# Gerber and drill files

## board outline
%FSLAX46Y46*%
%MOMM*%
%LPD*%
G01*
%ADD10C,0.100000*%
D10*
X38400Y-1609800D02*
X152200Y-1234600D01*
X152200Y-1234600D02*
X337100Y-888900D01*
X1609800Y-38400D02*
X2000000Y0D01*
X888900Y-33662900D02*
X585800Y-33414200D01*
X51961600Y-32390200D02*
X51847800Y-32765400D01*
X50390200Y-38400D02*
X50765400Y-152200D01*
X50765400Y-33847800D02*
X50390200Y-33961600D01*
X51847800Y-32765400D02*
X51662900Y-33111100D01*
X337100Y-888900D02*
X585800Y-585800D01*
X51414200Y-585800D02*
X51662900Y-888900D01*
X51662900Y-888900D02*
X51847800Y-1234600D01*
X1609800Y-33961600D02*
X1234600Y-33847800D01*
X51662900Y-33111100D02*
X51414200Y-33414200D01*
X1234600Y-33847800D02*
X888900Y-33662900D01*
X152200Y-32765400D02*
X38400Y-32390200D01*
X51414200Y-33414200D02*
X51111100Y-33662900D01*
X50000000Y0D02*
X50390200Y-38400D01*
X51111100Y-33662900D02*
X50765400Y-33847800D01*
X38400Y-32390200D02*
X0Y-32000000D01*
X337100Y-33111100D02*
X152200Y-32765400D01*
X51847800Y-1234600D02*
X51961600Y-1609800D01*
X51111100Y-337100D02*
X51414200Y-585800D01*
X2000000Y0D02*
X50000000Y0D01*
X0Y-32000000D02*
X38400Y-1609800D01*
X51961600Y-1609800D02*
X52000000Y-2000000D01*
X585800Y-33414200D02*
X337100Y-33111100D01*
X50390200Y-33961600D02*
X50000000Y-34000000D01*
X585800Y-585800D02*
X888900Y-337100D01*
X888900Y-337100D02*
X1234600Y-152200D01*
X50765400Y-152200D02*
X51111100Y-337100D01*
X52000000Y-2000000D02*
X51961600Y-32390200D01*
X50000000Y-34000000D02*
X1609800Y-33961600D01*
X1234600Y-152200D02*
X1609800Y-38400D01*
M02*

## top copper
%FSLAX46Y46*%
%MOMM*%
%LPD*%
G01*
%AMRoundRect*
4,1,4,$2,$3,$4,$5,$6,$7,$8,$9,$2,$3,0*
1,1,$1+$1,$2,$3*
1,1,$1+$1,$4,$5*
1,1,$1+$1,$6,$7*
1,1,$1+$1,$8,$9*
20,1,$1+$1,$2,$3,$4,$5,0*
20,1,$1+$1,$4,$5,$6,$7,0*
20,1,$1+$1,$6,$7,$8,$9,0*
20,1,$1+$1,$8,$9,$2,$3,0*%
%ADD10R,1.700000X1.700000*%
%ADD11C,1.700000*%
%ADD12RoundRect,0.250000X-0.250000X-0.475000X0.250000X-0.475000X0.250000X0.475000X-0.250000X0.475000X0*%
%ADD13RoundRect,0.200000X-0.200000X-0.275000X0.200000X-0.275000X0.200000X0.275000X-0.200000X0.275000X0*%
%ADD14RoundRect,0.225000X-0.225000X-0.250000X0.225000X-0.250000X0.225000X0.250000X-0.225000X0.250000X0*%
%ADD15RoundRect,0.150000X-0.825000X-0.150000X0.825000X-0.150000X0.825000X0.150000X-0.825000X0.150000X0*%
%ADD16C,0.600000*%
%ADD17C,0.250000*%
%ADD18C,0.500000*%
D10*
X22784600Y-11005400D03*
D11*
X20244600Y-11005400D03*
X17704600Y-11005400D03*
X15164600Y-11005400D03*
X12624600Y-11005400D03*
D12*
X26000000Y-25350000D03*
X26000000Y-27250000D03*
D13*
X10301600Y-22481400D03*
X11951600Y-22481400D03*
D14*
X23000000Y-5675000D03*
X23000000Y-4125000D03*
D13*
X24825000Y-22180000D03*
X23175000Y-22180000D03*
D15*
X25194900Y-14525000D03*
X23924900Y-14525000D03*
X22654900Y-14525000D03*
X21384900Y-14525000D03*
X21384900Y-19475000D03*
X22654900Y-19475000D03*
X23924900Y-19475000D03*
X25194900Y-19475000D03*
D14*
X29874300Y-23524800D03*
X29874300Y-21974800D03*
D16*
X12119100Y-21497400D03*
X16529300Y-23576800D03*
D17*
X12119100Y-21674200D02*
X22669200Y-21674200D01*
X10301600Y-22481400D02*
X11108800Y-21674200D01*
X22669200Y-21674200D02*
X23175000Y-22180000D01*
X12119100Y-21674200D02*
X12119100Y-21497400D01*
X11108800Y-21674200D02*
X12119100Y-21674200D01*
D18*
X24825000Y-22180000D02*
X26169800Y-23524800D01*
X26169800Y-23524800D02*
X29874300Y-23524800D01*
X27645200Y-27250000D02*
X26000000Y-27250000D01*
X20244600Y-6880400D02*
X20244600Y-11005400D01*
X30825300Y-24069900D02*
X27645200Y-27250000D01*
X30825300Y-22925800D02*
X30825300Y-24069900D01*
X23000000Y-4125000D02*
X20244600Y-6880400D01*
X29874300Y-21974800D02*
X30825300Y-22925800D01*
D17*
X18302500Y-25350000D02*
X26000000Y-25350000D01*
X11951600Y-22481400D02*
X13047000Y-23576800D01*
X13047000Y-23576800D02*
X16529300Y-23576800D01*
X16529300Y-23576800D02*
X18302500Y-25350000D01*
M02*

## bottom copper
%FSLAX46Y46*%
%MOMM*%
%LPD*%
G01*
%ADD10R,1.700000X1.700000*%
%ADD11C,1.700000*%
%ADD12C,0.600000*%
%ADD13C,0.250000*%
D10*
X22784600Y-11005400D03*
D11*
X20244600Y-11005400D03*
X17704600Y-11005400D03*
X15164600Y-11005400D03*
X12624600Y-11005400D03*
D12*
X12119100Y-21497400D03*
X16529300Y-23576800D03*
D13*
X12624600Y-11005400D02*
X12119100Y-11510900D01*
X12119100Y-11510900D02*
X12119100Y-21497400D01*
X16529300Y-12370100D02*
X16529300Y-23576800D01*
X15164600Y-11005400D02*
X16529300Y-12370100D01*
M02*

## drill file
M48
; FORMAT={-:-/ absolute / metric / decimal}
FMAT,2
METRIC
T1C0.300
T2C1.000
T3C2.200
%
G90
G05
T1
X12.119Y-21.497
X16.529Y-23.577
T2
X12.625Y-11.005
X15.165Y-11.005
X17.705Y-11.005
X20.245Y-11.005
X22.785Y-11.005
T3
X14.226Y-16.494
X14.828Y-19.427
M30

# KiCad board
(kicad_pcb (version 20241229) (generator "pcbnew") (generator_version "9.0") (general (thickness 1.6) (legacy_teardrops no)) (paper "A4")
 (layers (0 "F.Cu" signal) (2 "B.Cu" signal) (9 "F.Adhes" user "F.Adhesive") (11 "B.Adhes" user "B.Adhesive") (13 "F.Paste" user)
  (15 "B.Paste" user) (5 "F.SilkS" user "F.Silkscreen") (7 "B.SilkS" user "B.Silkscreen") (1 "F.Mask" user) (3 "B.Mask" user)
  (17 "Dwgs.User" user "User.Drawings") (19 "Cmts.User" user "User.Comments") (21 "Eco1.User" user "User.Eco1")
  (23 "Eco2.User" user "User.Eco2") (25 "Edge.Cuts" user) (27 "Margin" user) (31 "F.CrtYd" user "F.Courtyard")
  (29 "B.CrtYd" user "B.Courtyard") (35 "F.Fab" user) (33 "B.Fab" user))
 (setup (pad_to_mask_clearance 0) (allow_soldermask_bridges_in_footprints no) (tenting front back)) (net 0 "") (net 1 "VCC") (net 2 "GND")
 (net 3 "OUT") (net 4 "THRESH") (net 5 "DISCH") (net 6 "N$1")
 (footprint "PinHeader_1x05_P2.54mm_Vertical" (layer "F.Cu") (at 22.7846 11.0054 -90)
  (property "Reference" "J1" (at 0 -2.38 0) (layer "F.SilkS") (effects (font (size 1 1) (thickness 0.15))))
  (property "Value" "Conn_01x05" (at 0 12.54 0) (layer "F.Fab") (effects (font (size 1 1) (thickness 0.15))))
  (pad "1" thru_hole rect (at 0 0) (size 1.7 1.7) (drill 1) (layers "*.Cu" "*.Mask") (remove_unused_layers no) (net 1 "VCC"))
  (pad "2" thru_hole circle (at 0 2.54) (size 1.7 1.7) (drill 1) (layers "*.Cu" "*.Mask") (remove_unused_layers no) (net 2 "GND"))
  (pad "3" thru_hole circle (at 0 5.08) (size 1.7 1.7) (drill 1) (layers "*.Cu" "*.Mask") (remove_unused_layers no) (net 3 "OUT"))
  (pad "4" thru_hole circle (at 0 7.62) (size 1.7 1.7) (drill 1) (layers "*.Cu" "*.Mask") (remove_unused_layers no) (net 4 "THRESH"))
  (pad "5" thru_hole circle (at 0 10.16) (size 1.7 1.7) (drill 1) (layers "*.Cu" "*.Mask") (remove_unused_layers no) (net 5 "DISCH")))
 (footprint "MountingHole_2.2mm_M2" (layer "F.Cu") (at 14.8283 19.4265)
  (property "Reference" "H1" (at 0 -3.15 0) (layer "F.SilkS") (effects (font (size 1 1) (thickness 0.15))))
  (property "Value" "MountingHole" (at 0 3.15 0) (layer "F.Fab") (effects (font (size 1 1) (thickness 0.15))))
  (pad "" np_thru_hole circle (at 0 0) (size 2.2 2.2) (drill 2.2) (layers "*.Cu" "*.Mask")))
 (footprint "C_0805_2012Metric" (layer "F.Cu") (at 26 26.3 -90)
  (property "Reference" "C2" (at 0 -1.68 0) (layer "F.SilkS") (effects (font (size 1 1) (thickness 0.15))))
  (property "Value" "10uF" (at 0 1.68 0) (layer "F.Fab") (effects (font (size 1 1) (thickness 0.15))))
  (pad "1" smd roundrect (at -0.95 0) (size 1 1.45) (layers "F.Cu" "F.Mask" "F.Paste") (roundrect_rratio 0.25) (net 4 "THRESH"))
  (pad "2" smd roundrect (at 0.95 0) (size 1 1.45) (layers "F.Cu" "F.Mask" "F.Paste") (roundrect_rratio 0.25) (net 2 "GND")))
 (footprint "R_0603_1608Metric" (layer "F.Cu") (at 11.1266 22.4814)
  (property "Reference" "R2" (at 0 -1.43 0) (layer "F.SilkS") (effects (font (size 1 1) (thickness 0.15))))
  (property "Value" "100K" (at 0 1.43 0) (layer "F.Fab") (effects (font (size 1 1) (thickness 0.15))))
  (pad "1" smd roundrect (at -0.825 0) (size 0.8 0.95) (layers "F.Cu" "F.Mask" "F.Paste") (roundrect_rratio 0.25) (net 5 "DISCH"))
  (pad "2" smd roundrect (at 0.825 0) (size 0.8 0.95) (layers "F.Cu" "F.Mask" "F.Paste") (roundrect_rratio 0.25) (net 4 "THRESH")))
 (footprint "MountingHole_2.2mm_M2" (layer "F.Cu") (at 14.2257 16.4942)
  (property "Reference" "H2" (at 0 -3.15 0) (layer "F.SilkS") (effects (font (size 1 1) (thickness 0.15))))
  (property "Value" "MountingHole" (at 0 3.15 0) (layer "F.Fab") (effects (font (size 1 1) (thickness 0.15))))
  (pad "" np_thru_hole circle (at 0 0) (size 2.2 2.2) (drill 2.2) (layers "*.Cu" "*.Mask")))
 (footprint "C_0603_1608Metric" (layer "F.Cu") (at 23 4.9 90)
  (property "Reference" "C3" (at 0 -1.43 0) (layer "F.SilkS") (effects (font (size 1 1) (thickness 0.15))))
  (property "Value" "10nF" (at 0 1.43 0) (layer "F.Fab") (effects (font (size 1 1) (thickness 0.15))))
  (pad "1" smd roundrect (at -0.775 0) (size 0.9 0.95) (layers "F.Cu" "F.Mask" "F.Paste") (roundrect_rratio 0.25) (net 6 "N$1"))
  (pad "2" smd roundrect (at 0.775 0) (size 0.9 0.95) (layers "F.Cu" "F.Mask" "F.Paste") (roundrect_rratio 0.25) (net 2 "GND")))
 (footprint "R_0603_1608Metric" (layer "F.Cu") (at 24 22.18 180)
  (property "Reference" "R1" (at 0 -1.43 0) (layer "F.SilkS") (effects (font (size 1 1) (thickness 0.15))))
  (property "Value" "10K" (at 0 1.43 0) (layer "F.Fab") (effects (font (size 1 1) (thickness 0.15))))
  (pad "1" smd roundrect (at -0.825 0) (size 0.8 0.95) (layers "F.Cu" "F.Mask" "F.Paste") (roundrect_rratio 0.25) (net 1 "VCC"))
  (pad "2" smd roundrect (at 0.825 0) (size 0.8 0.95) (layers "F.Cu" "F.Mask" "F.Paste") (roundrect_rratio 0.25) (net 5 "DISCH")))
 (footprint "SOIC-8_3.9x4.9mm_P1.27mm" (layer "F.Cu") (at 23.2899 17 -90)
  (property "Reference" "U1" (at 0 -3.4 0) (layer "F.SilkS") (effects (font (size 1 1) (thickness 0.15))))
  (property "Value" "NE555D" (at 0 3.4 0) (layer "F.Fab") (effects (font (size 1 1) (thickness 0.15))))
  (pad "1" smd roundrect (at -2.475 -1.905) (size 1.95 0.6) (layers "F.Cu" "F.Mask" "F.Paste") (roundrect_rratio 0.25) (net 2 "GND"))
  (pad "2" smd roundrect (at -2.475 -0.635) (size 1.95 0.6) (layers "F.Cu" "F.Mask" "F.Paste") (roundrect_rratio 0.25) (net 4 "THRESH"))
  (pad "3" smd roundrect (at -2.475 0.635) (size 1.95 0.6) (layers "F.Cu" "F.Mask" "F.Paste") (roundrect_rratio 0.25) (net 3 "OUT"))
  (pad "4" smd roundrect (at -2.475 1.905) (size 1.95 0.6) (layers "F.Cu" "F.Mask" "F.Paste") (roundrect_rratio 0.25) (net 1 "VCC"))
  (pad "5" smd roundrect (at 2.475 1.905) (size 1.95 0.6) (layers "F.Cu" "F.Mask" "F.Paste") (roundrect_rratio 0.25) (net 6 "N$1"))
  (pad "6" smd roundrect (at 2.475 0.635) (size 1.95 0.6) (layers "F.Cu" "F.Mask" "F.Paste") (roundrect_rratio 0.25) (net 4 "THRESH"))
  (pad "7" smd roundrect (at 2.475 -0.635) (size 1.95 0.6) (layers "F.Cu" "F.Mask" "F.Paste") (roundrect_rratio 0.25) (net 5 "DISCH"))
  (pad "8" smd roundrect (at 2.475 -1.905) (size 1.95 0.6) (layers "F.Cu" "F.Mask" "F.Paste") (roundrect_rratio 0.25) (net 1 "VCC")))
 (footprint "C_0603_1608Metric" (layer "F.Cu") (at 29.8743 22.7498 90)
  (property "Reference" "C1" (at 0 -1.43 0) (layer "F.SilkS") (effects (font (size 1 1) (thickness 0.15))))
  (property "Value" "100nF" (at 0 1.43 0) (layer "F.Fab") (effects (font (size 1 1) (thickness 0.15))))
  (pad "1" smd roundrect (at -0.775 0) (size 0.9 0.95) (layers "F.Cu" "F.Mask" "F.Paste") (roundrect_rratio 0.25) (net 1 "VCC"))
  (pad "2" smd roundrect (at 0.775 0) (size 0.9 0.95) (layers "F.Cu" "F.Mask" "F.Paste") (roundrect_rratio 0.25) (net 2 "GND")))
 (gr_line (start 0.0384 1.6098) (end 0.1522 1.2346) (stroke (width 0.1) (type solid)) (layer "Edge.Cuts"))
 (gr_line (start 0.1522 1.2346) (end 0.3371 0.8889) (stroke (width 0.1) (type solid)) (layer "Edge.Cuts"))
 (gr_line (start 1.6098 0.0384) (end 2 0) (stroke (width 0.1) (type solid)) (layer "Edge.Cuts"))
 (gr_line (start 0.8889 33.6629) (end 0.5858 33.4142) (stroke (width 0.1) (type solid)) (layer "Edge.Cuts"))
 (gr_line (start 51.9616 32.3902) (end 51.8478 32.7654) (stroke (width 0.1) (type solid)) (layer "Edge.Cuts"))
 (gr_line (start 50.3902 0.0384) (end 50.7654 0.1522) (stroke (width 0.1) (type solid)) (layer "Edge.Cuts"))
 (gr_line (start 50.7654 33.8478) (end 50.3902 33.9616) (stroke (width 0.1) (type solid)) (layer "Edge.Cuts"))
 (gr_line (start 51.8478 32.7654) (end 51.6629 33.1111) (stroke (width 0.1) (type solid)) (layer "Edge.Cuts"))
 (gr_line (start 0.3371 0.8889) (end 0.5858 0.5858) (stroke (width 0.1) (type solid)) (layer "Edge.Cuts"))
 (gr_line (start 51.4142 0.5858) (end 51.6629 0.8889) (stroke (width 0.1) (type solid)) (layer "Edge.Cuts"))
 (gr_line (start 51.6629 0.8889) (end 51.8478 1.2346) (stroke (width 0.1) (type solid)) (layer "Edge.Cuts"))
 (gr_line (start 1.6098 33.9616) (end 1.2346 33.8478) (stroke (width 0.1) (type solid)) (layer "Edge.Cuts"))
 (gr_line (start 51.6629 33.1111) (end 51.4142 33.4142) (stroke (width 0.1) (type solid)) (layer "Edge.Cuts"))
 (gr_line (start 1.2346 33.8478) (end 0.8889 33.6629) (stroke (width 0.1) (type solid)) (layer "Edge.Cuts"))
 (gr_line (start 0.1522 32.7654) (end 0.0384 32.3902) (stroke (width 0.1) (type solid)) (layer "Edge.Cuts"))
 (gr_line (start 51.4142 33.4142) (end 51.1111 33.6629) (stroke (width 0.1) (type solid)) (layer "Edge.Cuts"))
 (gr_line (start 50 0) (end 50.3902 0.0384) (stroke (width 0.1) (type solid)) (layer "Edge.Cuts"))
 (gr_line (start 51.1111 33.6629) (end 50.7654 33.8478) (stroke (width 0.1) (type solid)) (layer "Edge.Cuts"))
 (gr_line (start 0.0384 32.3902) (end 0 32) (stroke (width 0.1) (type solid)) (layer "Edge.Cuts"))
 (gr_line (start 0.3371 33.1111) (end 0.1522 32.7654) (stroke (width 0.1) (type solid)) (layer "Edge.Cuts"))
 (gr_line (start 51.8478 1.2346) (end 51.9616 1.6098) (stroke (width 0.1) (type solid)) (layer "Edge.Cuts"))
 (gr_line (start 51.1111 0.3371) (end 51.4142 0.5858) (stroke (width 0.1) (type solid)) (layer "Edge.Cuts"))
 (gr_line (start 2 0) (end 50 0) (stroke (width 0.1) (type solid)) (layer "Edge.Cuts"))
 (gr_line (start 0 32) (end 0.0384 1.6098) (stroke (width 0.1) (type solid)) (layer "Edge.Cuts"))
 (gr_line (start 51.9616 1.6098) (end 52 2) (stroke (width 0.1) (type solid)) (layer "Edge.Cuts"))
 (gr_line (start 0.5858 33.4142) (end 0.3371 33.1111) (stroke (width 0.1) (type solid)) (layer "Edge.Cuts"))
 (gr_line (start 50.3902 33.9616) (end 50 34) (stroke (width 0.1) (type solid)) (layer "Edge.Cuts"))
 (gr_line (start 0.5858 0.5858) (end 0.8889 0.3371) (stroke (width 0.1) (type solid)) (layer "Edge.Cuts"))
 (gr_line (start 0.8889 0.3371) (end 1.2346 0.1522) (stroke (width 0.1) (type solid)) (layer "Edge.Cuts"))
 (gr_line (start 50.7654 0.1522) (end 51.1111 0.3371) (stroke (width 0.1) (type solid)) (layer "Edge.Cuts"))
 (gr_line (start 52 2) (end 51.9616 32.3902) (stroke (width 0.1) (type solid)) (layer "Edge.Cuts"))
 (gr_line (start 50 34) (end 1.6098 33.9616) (stroke (width 0.1) (type solid)) (layer "Edge.Cuts"))
 (gr_line (start 1.2346 0.1522) (end 1.6098 0.0384) (stroke (width 0.1) (type solid)) (layer "Edge.Cuts"))
 (segment (start 12.1191 21.6742) (end 22.6692 21.6742) (width 0.25) (layer "F.Cu") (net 5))
 (segment (start 10.3016 22.4814) (end 11.1088 21.6742) (width 0.25) (layer "F.Cu") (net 5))
 (segment (start 22.6692 21.6742) (end 23.175 22.18) (width 0.25) (layer "F.Cu") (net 5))
 (segment (start 12.1191 21.6742) (end 12.1191 21.4974) (width 0.25) (layer "F.Cu") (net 5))
 (segment (start 11.1088 21.6742) (end 12.1191 21.6742) (width 0.25) (layer "F.Cu") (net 5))
 (via (at 12.1191 21.4974) (size 0.6) (drill 0.3) (layers "F.Cu" "B.Cu") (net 5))
 (segment (start 12.6246 11.0054) (end 12.1191 11.5109) (width 0.25) (layer "B.Cu") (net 5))
 (segment (start 12.1191 11.5109) (end 12.1191 21.4974) (width 0.25) (layer "B.Cu") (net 5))
 (segment (start 24.825 22.18) (end 26.1698 23.5248) (width 0.5) (layer "F.Cu") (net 1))
 (segment (start 26.1698 23.5248) (end 29.8743 23.5248) (width 0.5) (layer "F.Cu") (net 1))
 (segment (start 27.6452 27.25) (end 26 27.25) (width 0.5) (layer "F.Cu") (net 2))
 (segment (start 20.2446 6.8804) (end 20.2446 11.0054) (width 0.5) (layer "F.Cu") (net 2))
 (segment (start 30.8253 24.0699) (end 27.6452 27.25) (width 0.5) (layer "F.Cu") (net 2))
 (segment (start 30.8253 22.9258) (end 30.8253 24.0699) (width 0.5) (layer "F.Cu") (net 2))
 (segment (start 23 4.125) (end 20.2446 6.8804) (width 0.5) (layer "F.Cu") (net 2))
 (segment (start 29.8743 21.9748) (end 30.8253 22.9258) (width 0.5) (layer "F.Cu") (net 2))
 (segment (start 18.3025 25.35) (end 26 25.35) (width 0.25) (layer "F.Cu") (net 4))
 (segment (start 11.9516 22.4814) (end 13.047 23.5768) (width 0.25) (layer "F.Cu") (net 4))
 (segment (start 13.047 23.5768) (end 16.5293 23.5768) (width 0.25) (layer "F.Cu") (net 4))
 (segment (start 16.5293 23.5768) (end 18.3025 25.35) (width 0.25) (layer "F.Cu") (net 4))
 (via (at 16.5293 23.5768) (size 0.6) (drill 0.3) (layers "F.Cu" "B.Cu") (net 4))
 (segment (start 16.5293 12.3701) (end 16.5293 23.5768) (width 0.25) (layer "B.Cu") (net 4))
 (segment (start 15.1646 11.0054) (end 16.5293 12.3701) (width 0.25) (layer "B.Cu") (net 4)))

